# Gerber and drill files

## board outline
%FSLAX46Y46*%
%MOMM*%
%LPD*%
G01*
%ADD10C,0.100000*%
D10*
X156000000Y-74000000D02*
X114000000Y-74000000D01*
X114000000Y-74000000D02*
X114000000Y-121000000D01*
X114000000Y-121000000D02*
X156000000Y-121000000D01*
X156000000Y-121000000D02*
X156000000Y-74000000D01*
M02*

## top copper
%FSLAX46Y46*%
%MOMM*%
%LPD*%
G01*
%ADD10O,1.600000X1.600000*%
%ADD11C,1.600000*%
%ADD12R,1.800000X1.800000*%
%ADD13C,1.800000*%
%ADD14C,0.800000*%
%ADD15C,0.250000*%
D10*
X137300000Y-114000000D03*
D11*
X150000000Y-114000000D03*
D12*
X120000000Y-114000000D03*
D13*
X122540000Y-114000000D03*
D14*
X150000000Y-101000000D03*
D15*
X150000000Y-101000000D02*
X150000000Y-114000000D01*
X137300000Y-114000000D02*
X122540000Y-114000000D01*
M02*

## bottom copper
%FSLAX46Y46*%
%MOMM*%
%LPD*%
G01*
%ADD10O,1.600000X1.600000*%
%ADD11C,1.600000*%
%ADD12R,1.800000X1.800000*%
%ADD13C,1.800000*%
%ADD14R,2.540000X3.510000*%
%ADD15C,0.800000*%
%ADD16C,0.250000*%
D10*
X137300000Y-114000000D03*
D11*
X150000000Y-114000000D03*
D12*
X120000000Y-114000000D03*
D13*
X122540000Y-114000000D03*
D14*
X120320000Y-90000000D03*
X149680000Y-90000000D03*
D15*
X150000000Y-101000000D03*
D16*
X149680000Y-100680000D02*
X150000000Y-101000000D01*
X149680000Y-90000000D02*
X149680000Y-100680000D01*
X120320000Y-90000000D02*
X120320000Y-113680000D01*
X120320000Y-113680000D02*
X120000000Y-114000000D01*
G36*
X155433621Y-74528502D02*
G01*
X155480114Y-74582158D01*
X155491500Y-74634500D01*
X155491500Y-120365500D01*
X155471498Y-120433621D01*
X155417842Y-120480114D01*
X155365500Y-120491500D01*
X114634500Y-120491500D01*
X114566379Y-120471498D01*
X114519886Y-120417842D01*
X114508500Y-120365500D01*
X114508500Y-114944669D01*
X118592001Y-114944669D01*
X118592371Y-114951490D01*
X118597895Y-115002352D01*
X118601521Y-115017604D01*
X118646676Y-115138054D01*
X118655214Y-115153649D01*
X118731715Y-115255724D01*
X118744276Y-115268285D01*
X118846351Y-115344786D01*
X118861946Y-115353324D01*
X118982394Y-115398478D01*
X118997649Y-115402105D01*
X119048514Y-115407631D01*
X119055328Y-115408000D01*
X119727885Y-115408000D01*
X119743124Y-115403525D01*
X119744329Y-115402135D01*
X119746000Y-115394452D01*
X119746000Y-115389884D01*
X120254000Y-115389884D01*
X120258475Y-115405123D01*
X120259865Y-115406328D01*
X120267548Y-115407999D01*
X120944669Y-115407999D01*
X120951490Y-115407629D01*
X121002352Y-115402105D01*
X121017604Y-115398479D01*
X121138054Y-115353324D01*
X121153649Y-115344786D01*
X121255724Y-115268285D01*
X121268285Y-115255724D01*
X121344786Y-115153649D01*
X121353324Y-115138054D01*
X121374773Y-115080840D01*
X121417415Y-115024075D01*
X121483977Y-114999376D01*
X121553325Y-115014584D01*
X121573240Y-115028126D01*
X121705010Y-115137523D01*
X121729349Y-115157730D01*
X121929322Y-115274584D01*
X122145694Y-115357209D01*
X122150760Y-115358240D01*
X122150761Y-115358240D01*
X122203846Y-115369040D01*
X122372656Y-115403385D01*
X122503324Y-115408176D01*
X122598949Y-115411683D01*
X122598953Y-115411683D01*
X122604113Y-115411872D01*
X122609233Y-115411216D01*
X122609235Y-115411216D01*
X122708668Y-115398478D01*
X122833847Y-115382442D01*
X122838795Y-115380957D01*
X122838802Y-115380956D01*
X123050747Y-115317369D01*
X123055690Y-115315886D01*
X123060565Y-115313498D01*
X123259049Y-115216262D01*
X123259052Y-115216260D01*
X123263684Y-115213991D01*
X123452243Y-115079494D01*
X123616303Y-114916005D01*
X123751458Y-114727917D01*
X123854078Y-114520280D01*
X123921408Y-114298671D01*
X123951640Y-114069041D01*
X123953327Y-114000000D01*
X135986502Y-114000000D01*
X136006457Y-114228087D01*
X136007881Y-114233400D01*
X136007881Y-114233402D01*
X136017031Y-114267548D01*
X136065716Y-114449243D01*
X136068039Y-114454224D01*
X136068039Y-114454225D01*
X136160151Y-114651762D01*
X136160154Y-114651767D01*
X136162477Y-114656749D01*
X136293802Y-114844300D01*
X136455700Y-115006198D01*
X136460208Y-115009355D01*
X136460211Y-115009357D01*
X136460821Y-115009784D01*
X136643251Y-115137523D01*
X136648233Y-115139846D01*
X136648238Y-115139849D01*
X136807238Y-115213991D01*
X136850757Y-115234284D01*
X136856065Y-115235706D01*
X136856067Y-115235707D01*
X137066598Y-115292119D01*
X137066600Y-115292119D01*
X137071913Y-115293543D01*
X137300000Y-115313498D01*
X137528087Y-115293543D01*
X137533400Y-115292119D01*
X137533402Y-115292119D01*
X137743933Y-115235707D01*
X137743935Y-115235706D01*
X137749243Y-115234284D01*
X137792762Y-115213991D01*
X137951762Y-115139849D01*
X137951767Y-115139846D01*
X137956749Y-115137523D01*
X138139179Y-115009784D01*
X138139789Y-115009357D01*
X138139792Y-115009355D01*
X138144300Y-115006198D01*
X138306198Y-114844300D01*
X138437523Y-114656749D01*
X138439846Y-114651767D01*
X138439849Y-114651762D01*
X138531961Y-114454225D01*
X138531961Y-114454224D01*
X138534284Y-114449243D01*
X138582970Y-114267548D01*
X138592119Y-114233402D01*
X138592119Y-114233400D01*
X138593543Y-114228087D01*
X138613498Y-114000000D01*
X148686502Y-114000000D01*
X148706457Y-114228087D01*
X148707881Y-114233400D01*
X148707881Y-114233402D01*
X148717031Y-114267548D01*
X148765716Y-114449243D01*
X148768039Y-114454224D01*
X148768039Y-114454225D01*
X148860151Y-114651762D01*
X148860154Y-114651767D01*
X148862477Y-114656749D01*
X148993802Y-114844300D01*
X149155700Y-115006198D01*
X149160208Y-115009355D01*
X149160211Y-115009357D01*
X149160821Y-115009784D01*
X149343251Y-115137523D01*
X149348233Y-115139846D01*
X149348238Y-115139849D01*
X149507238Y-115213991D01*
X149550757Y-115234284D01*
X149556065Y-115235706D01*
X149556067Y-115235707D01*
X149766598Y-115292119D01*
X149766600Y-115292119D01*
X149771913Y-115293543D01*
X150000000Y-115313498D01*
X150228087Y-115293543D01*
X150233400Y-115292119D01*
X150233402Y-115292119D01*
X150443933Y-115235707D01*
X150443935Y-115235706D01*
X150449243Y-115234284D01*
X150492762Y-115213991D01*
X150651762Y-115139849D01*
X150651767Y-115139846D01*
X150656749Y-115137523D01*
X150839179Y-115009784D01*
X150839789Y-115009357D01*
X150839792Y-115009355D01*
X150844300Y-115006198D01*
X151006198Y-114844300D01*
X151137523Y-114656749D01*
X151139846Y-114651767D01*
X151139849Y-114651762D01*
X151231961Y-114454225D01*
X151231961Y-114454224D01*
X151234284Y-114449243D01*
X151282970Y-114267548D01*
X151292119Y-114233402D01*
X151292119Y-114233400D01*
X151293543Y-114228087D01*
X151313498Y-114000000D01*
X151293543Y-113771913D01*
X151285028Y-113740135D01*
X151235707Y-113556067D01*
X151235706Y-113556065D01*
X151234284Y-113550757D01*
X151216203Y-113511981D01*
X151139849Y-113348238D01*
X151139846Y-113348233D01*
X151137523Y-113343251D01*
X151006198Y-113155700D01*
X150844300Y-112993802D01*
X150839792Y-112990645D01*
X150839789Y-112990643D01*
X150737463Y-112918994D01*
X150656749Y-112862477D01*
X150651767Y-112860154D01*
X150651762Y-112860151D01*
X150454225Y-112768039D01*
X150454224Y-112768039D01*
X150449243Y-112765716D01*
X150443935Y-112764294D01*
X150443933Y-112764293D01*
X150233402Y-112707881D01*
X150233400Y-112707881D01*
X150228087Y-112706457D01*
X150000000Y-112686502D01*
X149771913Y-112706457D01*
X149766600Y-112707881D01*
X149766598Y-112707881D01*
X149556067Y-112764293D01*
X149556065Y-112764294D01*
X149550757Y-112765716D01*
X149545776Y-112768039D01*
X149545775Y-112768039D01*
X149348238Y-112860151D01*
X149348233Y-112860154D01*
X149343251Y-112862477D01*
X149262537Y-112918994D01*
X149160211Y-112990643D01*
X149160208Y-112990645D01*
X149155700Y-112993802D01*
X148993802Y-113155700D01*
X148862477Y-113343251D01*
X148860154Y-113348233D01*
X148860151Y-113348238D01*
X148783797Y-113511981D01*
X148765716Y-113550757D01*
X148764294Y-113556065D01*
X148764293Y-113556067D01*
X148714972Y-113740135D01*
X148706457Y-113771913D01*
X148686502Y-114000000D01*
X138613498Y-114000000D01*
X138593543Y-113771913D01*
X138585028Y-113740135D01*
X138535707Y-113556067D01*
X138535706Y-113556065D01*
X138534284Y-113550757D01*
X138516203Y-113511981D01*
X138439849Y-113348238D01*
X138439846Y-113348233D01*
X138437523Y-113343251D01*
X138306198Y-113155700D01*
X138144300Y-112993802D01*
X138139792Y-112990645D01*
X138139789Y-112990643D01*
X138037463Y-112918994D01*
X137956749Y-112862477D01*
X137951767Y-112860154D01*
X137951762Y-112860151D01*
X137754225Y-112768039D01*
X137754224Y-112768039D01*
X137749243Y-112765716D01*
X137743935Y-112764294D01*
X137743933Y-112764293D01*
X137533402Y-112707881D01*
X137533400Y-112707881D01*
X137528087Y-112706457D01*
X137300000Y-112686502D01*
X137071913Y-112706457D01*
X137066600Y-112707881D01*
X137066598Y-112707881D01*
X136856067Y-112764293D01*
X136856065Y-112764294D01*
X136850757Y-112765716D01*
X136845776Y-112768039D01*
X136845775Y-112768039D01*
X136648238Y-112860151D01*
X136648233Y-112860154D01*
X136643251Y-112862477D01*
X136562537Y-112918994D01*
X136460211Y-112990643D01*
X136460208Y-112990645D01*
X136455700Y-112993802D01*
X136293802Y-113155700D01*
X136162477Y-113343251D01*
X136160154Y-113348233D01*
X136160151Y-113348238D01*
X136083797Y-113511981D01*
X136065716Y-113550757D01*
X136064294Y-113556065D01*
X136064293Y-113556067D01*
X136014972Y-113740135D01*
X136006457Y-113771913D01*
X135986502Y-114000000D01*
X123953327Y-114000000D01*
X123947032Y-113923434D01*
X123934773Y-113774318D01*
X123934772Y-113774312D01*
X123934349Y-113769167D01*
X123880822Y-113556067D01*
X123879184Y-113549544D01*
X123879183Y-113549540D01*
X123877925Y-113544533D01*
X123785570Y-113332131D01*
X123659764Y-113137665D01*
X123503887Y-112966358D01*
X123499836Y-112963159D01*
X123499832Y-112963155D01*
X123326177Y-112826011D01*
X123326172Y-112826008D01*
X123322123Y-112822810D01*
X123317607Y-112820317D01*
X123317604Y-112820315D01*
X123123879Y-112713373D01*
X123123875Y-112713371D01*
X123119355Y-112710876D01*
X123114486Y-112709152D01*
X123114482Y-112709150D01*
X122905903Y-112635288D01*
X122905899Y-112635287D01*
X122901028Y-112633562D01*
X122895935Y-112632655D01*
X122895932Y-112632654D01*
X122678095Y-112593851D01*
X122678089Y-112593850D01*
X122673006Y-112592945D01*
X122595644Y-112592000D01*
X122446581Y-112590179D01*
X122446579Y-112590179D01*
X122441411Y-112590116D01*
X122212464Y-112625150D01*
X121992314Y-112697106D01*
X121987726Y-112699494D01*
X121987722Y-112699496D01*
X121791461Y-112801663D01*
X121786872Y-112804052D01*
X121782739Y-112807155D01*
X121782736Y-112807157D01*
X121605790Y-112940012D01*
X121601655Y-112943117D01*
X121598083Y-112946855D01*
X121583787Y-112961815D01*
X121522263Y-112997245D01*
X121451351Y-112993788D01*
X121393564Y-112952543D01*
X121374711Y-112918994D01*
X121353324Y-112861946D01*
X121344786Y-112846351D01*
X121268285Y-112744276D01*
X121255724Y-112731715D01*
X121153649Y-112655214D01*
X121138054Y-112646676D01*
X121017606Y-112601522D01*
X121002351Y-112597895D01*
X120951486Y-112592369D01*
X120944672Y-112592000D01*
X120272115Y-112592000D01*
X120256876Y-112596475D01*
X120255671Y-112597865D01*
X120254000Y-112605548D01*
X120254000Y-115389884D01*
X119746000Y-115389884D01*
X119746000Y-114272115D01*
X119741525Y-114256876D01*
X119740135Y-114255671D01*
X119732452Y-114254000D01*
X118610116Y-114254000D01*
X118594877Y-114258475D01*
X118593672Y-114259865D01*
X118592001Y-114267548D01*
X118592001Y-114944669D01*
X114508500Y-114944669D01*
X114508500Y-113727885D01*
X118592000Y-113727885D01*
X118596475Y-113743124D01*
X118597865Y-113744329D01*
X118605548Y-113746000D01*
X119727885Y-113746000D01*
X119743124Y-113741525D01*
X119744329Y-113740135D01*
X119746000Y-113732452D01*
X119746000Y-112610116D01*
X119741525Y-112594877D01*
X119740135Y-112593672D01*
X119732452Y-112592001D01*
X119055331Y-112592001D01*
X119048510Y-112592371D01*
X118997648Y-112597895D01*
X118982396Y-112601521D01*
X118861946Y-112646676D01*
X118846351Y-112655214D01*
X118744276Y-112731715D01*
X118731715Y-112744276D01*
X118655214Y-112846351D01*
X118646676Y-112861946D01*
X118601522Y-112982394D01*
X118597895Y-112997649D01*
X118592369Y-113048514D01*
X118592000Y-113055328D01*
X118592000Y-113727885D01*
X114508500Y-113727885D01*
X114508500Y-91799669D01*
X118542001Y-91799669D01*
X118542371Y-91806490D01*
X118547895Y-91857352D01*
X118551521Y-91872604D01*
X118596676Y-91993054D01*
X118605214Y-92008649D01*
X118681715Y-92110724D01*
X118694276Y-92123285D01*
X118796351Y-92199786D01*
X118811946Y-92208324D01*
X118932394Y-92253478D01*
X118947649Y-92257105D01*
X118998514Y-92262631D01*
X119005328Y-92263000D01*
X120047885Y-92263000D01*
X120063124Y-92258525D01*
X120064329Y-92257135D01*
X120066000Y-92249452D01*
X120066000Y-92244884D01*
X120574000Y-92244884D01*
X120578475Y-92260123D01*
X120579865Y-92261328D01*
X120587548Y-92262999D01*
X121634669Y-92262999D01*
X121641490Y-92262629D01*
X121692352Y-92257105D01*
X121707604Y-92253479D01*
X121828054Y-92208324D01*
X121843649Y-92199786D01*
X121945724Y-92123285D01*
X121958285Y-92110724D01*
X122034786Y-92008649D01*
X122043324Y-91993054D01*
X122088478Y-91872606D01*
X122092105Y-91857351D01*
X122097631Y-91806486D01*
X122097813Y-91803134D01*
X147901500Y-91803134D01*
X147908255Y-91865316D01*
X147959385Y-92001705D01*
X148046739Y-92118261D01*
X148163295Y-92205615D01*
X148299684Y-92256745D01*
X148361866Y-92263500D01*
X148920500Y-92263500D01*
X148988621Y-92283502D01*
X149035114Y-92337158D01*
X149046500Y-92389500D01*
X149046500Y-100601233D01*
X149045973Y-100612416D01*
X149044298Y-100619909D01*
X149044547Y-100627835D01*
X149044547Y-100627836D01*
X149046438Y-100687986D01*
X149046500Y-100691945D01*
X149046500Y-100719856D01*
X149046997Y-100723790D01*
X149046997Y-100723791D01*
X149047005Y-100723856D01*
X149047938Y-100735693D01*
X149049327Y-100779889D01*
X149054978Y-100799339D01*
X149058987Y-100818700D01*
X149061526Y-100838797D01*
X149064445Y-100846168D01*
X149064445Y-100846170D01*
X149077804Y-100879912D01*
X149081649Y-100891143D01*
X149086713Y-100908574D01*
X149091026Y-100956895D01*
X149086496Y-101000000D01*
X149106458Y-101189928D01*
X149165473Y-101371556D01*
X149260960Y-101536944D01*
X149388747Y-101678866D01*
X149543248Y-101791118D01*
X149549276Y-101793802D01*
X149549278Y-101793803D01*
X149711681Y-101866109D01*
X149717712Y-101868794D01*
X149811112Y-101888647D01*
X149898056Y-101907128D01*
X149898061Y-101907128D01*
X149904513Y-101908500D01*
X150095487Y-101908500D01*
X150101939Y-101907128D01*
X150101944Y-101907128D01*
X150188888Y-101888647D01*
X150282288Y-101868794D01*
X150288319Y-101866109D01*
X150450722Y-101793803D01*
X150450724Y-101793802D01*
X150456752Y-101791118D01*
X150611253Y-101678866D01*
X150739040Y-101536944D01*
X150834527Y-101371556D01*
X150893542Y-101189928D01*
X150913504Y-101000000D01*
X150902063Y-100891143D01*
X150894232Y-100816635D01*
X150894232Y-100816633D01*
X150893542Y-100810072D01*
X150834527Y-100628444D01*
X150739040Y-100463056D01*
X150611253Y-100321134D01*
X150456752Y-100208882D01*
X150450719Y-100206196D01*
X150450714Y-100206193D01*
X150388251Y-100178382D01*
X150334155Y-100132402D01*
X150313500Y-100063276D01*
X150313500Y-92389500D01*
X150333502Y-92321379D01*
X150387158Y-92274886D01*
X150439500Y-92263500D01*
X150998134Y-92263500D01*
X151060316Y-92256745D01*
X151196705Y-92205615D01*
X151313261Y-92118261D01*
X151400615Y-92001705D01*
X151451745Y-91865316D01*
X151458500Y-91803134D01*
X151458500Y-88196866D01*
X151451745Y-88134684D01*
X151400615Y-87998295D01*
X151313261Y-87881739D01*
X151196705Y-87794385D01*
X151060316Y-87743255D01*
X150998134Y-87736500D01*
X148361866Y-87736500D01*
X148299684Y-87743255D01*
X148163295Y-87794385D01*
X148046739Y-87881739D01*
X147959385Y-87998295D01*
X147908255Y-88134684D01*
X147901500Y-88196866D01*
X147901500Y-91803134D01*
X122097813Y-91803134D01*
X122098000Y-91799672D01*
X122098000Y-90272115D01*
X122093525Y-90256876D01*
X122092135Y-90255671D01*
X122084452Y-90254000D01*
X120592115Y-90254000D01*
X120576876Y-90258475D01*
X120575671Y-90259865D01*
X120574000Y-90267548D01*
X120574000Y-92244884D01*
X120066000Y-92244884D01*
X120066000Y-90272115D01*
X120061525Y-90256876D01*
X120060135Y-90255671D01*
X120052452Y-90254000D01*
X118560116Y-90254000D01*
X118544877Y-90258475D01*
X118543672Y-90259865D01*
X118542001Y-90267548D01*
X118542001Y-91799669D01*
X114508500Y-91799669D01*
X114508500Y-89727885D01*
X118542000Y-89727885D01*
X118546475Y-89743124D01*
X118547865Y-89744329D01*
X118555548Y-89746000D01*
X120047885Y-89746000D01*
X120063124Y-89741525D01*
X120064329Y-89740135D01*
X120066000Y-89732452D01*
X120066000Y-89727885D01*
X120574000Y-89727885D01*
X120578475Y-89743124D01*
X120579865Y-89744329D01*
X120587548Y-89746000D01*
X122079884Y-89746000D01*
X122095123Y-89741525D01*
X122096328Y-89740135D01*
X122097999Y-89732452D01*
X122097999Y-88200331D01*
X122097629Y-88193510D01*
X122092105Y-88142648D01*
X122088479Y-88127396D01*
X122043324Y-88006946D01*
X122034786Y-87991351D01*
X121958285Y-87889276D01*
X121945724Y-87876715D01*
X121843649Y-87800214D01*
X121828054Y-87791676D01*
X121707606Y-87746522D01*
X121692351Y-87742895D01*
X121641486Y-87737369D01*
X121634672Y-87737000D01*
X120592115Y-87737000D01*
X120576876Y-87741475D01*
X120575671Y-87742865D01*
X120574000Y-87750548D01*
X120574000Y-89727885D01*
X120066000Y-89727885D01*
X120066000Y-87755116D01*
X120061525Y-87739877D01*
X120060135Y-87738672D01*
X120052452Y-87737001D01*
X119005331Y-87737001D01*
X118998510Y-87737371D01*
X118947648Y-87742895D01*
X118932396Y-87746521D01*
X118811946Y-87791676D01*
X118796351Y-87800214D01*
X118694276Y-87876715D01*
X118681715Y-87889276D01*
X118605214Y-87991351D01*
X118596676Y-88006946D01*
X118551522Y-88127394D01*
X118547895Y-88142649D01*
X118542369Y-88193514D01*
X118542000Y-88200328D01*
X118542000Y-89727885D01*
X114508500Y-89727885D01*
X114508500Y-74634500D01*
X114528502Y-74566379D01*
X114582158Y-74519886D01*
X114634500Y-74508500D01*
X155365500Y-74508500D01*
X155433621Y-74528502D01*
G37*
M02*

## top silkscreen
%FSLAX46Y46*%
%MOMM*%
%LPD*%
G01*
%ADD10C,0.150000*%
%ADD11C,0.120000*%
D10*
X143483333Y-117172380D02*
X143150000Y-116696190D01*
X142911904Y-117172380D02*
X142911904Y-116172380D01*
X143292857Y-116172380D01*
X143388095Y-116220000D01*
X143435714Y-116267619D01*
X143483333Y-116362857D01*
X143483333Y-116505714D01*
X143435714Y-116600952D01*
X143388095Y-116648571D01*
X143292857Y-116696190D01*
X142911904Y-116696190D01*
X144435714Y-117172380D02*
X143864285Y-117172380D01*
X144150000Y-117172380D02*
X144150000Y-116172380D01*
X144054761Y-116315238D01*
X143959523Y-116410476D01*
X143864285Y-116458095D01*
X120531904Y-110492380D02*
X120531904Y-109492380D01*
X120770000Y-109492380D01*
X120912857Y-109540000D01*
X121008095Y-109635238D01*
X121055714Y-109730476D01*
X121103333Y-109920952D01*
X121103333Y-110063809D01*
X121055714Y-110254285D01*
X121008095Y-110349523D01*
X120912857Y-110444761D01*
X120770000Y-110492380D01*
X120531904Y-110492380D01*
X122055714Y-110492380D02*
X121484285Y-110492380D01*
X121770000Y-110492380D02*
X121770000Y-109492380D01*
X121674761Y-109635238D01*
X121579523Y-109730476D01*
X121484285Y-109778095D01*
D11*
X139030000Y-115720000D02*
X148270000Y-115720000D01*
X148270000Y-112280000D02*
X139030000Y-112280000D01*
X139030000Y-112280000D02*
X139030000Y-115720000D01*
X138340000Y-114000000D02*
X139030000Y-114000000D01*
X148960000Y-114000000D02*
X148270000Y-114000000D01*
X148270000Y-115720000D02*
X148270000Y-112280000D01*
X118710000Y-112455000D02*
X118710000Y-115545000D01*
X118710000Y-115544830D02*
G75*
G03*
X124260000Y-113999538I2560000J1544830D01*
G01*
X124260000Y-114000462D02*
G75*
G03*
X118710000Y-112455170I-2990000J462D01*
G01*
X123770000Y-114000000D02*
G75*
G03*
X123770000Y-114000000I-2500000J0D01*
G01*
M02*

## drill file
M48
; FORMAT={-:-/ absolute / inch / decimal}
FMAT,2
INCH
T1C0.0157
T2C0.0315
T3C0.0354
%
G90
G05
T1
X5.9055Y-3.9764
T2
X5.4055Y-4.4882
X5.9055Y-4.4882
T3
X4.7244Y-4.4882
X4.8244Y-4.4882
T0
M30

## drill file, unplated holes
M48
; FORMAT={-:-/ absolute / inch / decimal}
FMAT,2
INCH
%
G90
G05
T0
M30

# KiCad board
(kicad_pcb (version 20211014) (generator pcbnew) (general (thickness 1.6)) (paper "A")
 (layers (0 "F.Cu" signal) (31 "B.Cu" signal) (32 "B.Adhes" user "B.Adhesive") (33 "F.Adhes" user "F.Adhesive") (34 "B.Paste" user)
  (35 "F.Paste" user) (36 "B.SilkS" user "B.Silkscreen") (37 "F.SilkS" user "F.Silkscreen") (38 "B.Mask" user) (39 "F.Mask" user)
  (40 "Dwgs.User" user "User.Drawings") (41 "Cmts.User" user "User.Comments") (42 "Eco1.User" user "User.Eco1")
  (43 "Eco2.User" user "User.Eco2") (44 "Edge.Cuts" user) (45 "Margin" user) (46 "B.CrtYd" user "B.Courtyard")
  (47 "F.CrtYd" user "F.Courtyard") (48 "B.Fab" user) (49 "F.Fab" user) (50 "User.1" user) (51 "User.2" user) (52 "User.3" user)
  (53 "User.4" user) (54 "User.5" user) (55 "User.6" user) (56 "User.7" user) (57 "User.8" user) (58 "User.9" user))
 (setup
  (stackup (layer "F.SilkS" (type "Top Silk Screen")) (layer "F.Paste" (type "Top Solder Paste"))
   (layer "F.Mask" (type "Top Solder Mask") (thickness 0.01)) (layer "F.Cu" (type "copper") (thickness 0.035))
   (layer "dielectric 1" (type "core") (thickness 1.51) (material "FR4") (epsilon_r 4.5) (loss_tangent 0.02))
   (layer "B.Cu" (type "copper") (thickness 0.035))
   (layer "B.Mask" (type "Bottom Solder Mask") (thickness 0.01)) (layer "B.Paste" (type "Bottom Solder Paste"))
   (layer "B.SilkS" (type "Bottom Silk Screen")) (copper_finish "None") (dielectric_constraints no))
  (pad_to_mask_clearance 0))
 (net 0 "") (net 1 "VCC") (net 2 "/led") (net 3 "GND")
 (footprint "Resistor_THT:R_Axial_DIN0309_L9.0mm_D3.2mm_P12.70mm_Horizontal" (layer "F.Cu") (at 150 114 180)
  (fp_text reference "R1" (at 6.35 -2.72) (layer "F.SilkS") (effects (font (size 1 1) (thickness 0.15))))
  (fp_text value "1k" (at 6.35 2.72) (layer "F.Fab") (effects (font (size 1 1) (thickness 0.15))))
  (fp_line (start 10.97 1.72) (end 10.97 -1.72) (layer "F.SilkS") (width 0.12))
  (fp_line (start 1.73 1.72) (end 10.97 1.72) (layer "F.SilkS") (width 0.12))
  (fp_line (start 1.04 0) (end 1.73 0) (layer "F.SilkS") (width 0.12))
  (fp_line (start 1.73 -1.72) (end 1.73 1.72) (layer "F.SilkS") (width 0.12))
  (fp_line (start 10.97 -1.72) (end 1.73 -1.72) (layer "F.SilkS") (width 0.12))
  (fp_line (start 11.66 0) (end 10.97 0) (layer "F.SilkS") (width 0.12))
  (pad "1" thru_hole circle (at 0 0 180) (size 1.6 1.6) (drill 0.8) (layers *.Cu *.Mask) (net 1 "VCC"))
  (pad "2" thru_hole oval (at 12.7 0 180) (size 1.6 1.6) (drill 0.8) (layers *.Cu *.Mask) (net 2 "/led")))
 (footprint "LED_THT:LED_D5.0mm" (layer "F.Cu") (at 120 114)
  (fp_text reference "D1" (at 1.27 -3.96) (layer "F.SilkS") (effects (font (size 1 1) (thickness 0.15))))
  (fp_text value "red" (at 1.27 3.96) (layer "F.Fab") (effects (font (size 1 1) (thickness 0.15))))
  (fp_line (start -1.29 -1.545) (end -1.29 1.545) (layer "F.SilkS") (width 0.12))
  (fp_arc (start -1.29 -1.54483) (mid 2.072002 -2.880433) (end 4.26 0.000462) (layer "F.SilkS") (width 0.12))
  (fp_arc (start 4.26 -0.000462) (mid 2.072002 2.880433) (end -1.29 1.54483) (layer "F.SilkS") (width 0.12))
  (fp_circle (center 1.27 0) (end 3.77 0) (layer "F.SilkS") (width 0.12) (fill none))
  (pad "1" thru_hole rect (at 0 0) (size 1.8 1.8) (drill 0.9) (layers *.Cu *.Mask) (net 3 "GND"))
  (pad "2" thru_hole circle (at 2.54 0) (size 1.8 1.8) (drill 0.9) (layers *.Cu *.Mask) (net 2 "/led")))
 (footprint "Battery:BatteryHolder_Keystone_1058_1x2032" (layer "B.Cu") (at 135 90 180)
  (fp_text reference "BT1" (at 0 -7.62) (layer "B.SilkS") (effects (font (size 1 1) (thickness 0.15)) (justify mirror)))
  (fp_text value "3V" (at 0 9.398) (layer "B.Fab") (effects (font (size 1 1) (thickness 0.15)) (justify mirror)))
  (pad "1" smd rect (at -14.68 0 180) (size 2.54 3.51) (layers "B.Cu" "B.Paste" "B.Mask") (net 1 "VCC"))
  (pad "2" smd rect (at 14.68 0 180) (size 2.54 3.51) (layers "B.Cu" "B.Paste" "B.Mask") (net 3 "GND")))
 (gr_rect (start 156 74) (end 114 121) (layer "Edge.Cuts") (width 0.1) (fill none))
 (segment (start 150 101) (end 150 114) (width 0.25) (layer "F.Cu") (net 1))
 (via (at 150 101) (size 0.8) (drill 0.4) (layers "F.Cu" "B.Cu") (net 1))
 (segment (start 149.68 100.68) (end 150 101) (width 0.25) (layer "B.Cu") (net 1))
 (segment (start 149.68 90) (end 149.68 100.68) (width 0.25) (layer "B.Cu") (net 1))
 (segment (start 120.32 90) (end 120.32 113.68) (width 0.25) (layer "B.Cu") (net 3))
 (segment (start 120.32 113.68) (end 120 114) (width 0.25) (layer "B.Cu") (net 3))
 (segment (start 137.3 114) (end 122.54 114) (width 0.25) (layer "F.Cu") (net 2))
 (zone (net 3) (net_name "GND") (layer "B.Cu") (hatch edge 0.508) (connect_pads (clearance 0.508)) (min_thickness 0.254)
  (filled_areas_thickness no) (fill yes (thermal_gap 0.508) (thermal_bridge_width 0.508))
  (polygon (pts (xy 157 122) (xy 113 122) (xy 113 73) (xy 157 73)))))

